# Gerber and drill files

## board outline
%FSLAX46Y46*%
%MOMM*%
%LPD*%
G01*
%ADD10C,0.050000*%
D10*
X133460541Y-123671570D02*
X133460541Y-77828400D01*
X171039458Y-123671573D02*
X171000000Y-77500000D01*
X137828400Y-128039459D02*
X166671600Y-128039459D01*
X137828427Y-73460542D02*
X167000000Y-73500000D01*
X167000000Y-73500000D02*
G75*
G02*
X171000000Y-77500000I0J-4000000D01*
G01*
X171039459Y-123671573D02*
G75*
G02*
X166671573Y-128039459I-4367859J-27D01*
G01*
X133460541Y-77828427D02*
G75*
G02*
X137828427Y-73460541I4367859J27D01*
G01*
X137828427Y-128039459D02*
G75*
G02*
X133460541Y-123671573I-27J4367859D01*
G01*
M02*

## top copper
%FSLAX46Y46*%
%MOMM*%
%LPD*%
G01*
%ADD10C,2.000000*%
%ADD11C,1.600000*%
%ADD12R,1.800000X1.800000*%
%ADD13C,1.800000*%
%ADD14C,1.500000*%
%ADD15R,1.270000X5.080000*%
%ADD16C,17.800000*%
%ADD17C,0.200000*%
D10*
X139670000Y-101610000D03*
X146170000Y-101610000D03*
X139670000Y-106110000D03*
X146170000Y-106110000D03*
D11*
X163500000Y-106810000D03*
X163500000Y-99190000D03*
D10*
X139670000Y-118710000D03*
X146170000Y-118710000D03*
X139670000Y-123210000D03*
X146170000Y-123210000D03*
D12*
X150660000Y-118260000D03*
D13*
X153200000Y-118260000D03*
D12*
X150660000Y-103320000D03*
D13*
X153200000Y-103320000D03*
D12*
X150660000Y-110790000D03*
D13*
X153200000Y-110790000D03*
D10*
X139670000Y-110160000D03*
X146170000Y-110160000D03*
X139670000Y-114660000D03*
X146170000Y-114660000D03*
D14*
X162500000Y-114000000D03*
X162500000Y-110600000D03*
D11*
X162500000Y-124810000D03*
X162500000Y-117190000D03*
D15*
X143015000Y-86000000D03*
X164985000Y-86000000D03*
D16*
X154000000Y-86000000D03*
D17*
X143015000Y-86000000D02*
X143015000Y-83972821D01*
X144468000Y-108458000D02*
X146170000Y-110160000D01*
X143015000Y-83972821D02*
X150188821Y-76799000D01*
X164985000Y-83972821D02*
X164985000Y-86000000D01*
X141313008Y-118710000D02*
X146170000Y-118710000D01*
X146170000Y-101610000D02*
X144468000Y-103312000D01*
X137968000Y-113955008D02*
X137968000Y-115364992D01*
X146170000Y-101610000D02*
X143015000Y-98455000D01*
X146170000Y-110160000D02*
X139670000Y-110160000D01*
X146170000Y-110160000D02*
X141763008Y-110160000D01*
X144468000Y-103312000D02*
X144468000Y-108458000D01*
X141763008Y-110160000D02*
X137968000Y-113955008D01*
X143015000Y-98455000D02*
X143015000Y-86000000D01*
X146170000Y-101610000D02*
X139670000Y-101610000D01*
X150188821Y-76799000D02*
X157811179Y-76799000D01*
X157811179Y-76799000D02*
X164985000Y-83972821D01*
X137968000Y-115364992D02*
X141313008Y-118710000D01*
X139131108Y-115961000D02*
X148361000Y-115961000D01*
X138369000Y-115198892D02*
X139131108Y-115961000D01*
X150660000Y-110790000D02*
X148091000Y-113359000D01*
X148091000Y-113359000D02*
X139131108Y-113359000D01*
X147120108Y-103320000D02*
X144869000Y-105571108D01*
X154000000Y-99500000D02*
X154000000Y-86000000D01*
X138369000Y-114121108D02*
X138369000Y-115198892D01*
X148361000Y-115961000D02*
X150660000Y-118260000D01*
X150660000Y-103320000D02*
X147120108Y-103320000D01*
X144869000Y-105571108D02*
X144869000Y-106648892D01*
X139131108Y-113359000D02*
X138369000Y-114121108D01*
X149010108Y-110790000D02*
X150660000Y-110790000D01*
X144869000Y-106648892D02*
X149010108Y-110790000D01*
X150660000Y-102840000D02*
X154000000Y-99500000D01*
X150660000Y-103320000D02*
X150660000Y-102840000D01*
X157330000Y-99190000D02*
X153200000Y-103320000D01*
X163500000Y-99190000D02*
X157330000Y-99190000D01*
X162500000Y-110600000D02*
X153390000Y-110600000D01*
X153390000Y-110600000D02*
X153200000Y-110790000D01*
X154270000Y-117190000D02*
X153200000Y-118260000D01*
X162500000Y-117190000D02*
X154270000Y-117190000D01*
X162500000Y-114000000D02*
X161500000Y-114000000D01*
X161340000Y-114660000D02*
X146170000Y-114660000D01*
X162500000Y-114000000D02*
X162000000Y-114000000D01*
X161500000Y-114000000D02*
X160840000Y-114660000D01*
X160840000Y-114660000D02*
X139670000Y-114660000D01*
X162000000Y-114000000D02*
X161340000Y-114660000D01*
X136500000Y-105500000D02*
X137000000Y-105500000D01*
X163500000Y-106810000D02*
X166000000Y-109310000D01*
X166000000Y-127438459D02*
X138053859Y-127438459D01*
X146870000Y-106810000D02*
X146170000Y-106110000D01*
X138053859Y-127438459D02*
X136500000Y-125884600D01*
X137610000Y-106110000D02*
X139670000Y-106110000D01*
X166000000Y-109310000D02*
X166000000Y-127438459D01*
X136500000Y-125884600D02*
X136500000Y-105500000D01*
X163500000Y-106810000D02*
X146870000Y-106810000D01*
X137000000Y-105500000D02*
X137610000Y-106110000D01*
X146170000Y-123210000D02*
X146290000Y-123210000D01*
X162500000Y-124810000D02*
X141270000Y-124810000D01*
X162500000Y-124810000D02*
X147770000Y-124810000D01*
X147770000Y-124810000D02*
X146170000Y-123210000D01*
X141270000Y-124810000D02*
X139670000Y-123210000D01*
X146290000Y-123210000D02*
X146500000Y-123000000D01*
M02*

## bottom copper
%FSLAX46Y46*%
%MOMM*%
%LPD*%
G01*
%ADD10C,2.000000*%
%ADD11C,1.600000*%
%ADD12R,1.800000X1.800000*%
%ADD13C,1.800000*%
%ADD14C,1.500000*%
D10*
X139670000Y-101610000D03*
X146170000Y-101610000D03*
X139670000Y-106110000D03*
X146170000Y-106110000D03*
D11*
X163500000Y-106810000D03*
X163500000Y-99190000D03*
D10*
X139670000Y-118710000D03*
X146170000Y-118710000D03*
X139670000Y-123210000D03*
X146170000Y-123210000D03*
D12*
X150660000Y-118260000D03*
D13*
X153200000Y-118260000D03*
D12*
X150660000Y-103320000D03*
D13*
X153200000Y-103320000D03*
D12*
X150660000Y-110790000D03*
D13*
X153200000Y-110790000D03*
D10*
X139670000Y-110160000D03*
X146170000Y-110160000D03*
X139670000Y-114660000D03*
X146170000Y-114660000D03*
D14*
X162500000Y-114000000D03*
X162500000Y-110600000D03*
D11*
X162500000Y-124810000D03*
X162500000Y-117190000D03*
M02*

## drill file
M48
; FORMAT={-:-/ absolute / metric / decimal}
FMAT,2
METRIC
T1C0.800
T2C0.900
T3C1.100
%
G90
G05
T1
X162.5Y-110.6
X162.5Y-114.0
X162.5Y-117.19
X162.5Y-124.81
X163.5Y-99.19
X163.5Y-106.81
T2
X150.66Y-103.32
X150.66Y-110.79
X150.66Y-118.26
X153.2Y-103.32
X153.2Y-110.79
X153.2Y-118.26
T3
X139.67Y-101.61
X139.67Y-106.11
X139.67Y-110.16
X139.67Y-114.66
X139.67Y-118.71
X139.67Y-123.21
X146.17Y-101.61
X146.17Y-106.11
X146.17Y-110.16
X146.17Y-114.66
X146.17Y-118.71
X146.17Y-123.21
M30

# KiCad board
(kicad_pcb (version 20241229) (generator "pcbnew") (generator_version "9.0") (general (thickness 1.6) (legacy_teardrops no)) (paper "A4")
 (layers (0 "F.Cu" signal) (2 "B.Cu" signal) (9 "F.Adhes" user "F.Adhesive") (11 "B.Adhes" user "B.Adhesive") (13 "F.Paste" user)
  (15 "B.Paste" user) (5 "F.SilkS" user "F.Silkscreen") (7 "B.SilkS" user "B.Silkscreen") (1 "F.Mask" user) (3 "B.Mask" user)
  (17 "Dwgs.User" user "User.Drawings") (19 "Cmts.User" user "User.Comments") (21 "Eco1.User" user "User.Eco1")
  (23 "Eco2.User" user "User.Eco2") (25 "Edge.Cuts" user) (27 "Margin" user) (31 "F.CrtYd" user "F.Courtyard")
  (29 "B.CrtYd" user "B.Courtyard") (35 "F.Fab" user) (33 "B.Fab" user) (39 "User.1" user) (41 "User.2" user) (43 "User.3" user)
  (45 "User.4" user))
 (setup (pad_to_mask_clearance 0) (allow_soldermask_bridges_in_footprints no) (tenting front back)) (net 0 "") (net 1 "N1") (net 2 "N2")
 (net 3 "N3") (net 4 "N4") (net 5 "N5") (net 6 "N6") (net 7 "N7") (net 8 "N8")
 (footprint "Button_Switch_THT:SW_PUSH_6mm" (layer "F.Cu") (at 139.67 101.61)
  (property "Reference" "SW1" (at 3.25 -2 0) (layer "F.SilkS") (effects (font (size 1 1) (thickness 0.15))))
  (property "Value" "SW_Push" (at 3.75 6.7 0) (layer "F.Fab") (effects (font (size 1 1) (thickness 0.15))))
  (pad "1" thru_hole circle (at 0 0 90) (size 2 2) (drill 1.1) (layers "*.Cu" "*.Mask") (remove_unused_layers no) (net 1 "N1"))
  (pad "1" thru_hole circle (at 6.5 0 90) (size 2 2) (drill 1.1) (layers "*.Cu" "*.Mask") (remove_unused_layers no) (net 1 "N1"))
  (pad "2" thru_hole circle (at 0 4.5 90) (size 2 2) (drill 1.1) (layers "*.Cu" "*.Mask") (remove_unused_layers no) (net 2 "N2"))
  (pad "2" thru_hole circle (at 6.5 4.5 90) (size 2 2) (drill 1.1) (layers "*.Cu" "*.Mask") (remove_unused_layers no) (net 2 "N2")))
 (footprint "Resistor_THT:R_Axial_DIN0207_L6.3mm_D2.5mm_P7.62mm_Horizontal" (layer "F.Cu") (at 163.5 106.81 90)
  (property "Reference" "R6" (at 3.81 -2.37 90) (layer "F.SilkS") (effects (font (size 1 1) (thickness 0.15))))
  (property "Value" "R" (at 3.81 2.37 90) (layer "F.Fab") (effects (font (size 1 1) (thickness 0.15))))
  (pad "1" thru_hole circle (at 0 0 90) (size 1.6 1.6) (drill 0.8) (layers "*.Cu" "*.Mask") (remove_unused_layers no) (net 2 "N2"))
  (pad "2" thru_hole circle (at 7.62 0 90) (size 1.6 1.6) (drill 0.8) (layers "*.Cu" "*.Mask") (remove_unused_layers no) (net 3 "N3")))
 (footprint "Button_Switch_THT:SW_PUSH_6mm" (layer "F.Cu") (at 139.67 118.71)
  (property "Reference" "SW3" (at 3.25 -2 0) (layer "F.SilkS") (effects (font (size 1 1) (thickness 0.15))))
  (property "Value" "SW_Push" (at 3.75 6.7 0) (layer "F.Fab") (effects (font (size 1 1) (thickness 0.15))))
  (pad "1" thru_hole circle (at 0 0 90) (size 2 2) (drill 1.1) (layers "*.Cu" "*.Mask") (remove_unused_layers no) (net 1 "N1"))
  (pad "1" thru_hole circle (at 6.5 0 90) (size 2 2) (drill 1.1) (layers "*.Cu" "*.Mask") (remove_unused_layers no) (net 1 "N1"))
  (pad "2" thru_hole circle (at 0 4.5 90) (size 2 2) (drill 1.1) (layers "*.Cu" "*.Mask") (remove_unused_layers no) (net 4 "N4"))
  (pad "2" thru_hole circle (at 6.5 4.5 90) (size 2 2) (drill 1.1) (layers "*.Cu" "*.Mask") (remove_unused_layers no) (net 4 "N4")))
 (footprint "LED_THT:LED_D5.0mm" (layer "F.Cu") (at 150.66 118.26)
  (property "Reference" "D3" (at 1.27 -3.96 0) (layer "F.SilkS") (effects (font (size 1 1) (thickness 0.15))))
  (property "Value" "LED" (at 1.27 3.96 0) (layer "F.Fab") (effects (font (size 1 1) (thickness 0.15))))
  (pad "1" thru_hole rect (at 0 0) (size 1.8 1.8) (drill 0.9) (layers "*.Cu" "*.Mask") (remove_unused_layers no) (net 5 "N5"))
  (pad "2" thru_hole circle (at 2.54 0) (size 1.8 1.8) (drill 0.9) (layers "*.Cu" "*.Mask") (remove_unused_layers no) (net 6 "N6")))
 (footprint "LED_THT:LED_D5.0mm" (layer "F.Cu") (at 150.66 103.32)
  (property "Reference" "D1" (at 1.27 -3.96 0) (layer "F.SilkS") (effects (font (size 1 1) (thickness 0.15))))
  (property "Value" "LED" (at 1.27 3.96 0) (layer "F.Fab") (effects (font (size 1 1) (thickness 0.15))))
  (pad "1" thru_hole rect (at 0 0) (size 1.8 1.8) (drill 0.9) (layers "*.Cu" "*.Mask") (remove_unused_layers no) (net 5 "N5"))
  (pad "2" thru_hole circle (at 2.54 0) (size 1.8 1.8) (drill 0.9) (layers "*.Cu" "*.Mask") (remove_unused_layers no) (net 3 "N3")))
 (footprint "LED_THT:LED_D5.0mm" (layer "F.Cu") (at 150.66 110.79)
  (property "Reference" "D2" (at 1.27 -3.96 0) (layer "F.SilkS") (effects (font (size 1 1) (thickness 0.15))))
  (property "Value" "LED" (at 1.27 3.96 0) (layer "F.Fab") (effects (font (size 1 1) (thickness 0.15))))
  (pad "1" thru_hole rect (at 0 0) (size 1.8 1.8) (drill 0.9) (layers "*.Cu" "*.Mask") (remove_unused_layers no) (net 5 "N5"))
  (pad "2" thru_hole circle (at 2.54 0) (size 1.8 1.8) (drill 0.9) (layers "*.Cu" "*.Mask") (remove_unused_layers no) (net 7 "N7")))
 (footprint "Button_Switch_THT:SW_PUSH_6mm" (layer "F.Cu") (at 139.67 110.16)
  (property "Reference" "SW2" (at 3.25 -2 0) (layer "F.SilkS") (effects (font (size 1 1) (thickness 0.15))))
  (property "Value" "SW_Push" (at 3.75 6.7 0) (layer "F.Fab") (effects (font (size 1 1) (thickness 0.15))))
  (pad "1" thru_hole circle (at 0 0 90) (size 2 2) (drill 1.1) (layers "*.Cu" "*.Mask") (remove_unused_layers no) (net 1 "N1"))
  (pad "1" thru_hole circle (at 6.5 0 90) (size 2 2) (drill 1.1) (layers "*.Cu" "*.Mask") (remove_unused_layers no) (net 1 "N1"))
  (pad "2" thru_hole circle (at 0 4.5 90) (size 2 2) (drill 1.1) (layers "*.Cu" "*.Mask") (remove_unused_layers no) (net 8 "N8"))
  (pad "2" thru_hole circle (at 6.5 4.5 90) (size 2 2) (drill 1.1) (layers "*.Cu" "*.Mask") (remove_unused_layers no) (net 8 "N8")))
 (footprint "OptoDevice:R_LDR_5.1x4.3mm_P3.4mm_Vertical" (layer "F.Cu") (at 162.5 114 90)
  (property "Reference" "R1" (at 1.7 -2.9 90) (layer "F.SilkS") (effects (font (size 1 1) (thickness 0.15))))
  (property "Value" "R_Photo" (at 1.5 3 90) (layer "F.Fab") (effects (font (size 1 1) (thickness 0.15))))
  (pad "1" thru_hole circle (at 0 0 90) (size 1.5 1.5) (drill 0.8) (layers "*.Cu" "*.Mask") (remove_unused_layers no) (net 8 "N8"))
  (pad "2" thru_hole circle (at 3.4 0 90) (size 1.5 1.5) (drill 0.8) (layers "*.Cu" "*.Mask") (remove_unused_layers no) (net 7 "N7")))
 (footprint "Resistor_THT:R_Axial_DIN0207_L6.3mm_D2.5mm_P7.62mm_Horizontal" (layer "F.Cu") (at 162.5 124.81 90)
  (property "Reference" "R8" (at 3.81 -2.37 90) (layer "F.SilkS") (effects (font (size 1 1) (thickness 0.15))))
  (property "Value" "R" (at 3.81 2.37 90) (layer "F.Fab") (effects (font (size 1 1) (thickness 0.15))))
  (pad "1" thru_hole circle (at 0 0 90) (size 1.6 1.6) (drill 0.8) (layers "*.Cu" "*.Mask") (remove_unused_layers no) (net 4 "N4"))
  (pad "2" thru_hole circle (at 7.62 0 90) (size 1.6 1.6) (drill 0.8) (layers "*.Cu" "*.Mask") (remove_unused_layers no) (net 6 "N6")))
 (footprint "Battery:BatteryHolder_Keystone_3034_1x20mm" (layer "F.Cu") (at 154 86)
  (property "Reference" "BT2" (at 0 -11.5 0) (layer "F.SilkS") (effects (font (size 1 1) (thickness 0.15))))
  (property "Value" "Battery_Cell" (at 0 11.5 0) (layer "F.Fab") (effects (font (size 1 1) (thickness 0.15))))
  (pad "1" smd rect (at -10.985 0) (size 1.27 5.08) (layers "F.Cu" "F.Mask" "F.Paste") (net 1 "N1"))
  (pad "1" smd rect (at 10.985 0) (size 1.27 5.08) (layers "F.Cu" "F.Mask" "F.Paste") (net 1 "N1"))
  (pad "2" smd circle (at 0 0) (size 17.8 17.8) (layers "F.Cu" "F.Mask") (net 5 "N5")))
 (gr_line (start 133.460541 123.67157) (end 133.460541 77.8284) (stroke (width 0.05) (type default)) (layer "Edge.Cuts"))
 (gr_line (start 171.039458 123.671573) (end 171 77.5) (stroke (width 0.05) (type default)) (layer "Edge.Cuts"))
 (gr_line (start 137.8284 128.039459) (end 166.6716 128.039459) (stroke (width 0.05) (type default)) (layer "Edge.Cuts"))
 (gr_line (start 137.828427 73.460542) (end 167 73.5) (stroke (width 0.05) (type default)) (layer "Edge.Cuts"))
 (gr_arc (start 167 73.5) (mid 169.828427 74.671573) (end 171 77.5) (stroke (width 0.05) (type default)) (layer "Edge.Cuts"))
 (gr_arc (start 171.039459 123.671573) (mid 169.760135 126.760135) (end 166.671573 128.039459) (stroke (width 0.05) (type default))
  (layer "Edge.Cuts"))
 (gr_arc (start 133.460541 77.828427) (mid 134.739865 74.739865) (end 137.828427 73.460541) (stroke (width 0.05) (type default))
  (layer "Edge.Cuts"))
 (gr_arc (start 137.828427 128.039459) (mid 134.739865 126.760135) (end 133.460541 123.671573) (stroke (width 0.05) (type default))
  (layer "Edge.Cuts"))
 (segment (start 143.015 86) (end 143.015 83.972821) (width 0.2) (layer "F.Cu") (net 1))
 (segment (start 144.468 108.458) (end 146.17 110.16) (width 0.2) (layer "F.Cu") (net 1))
 (segment (start 143.015 83.972821) (end 150.188821 76.799) (width 0.2) (layer "F.Cu") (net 1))
 (segment (start 164.985 83.972821) (end 164.985 86) (width 0.2) (layer "F.Cu") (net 1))
 (segment (start 141.313008 118.71) (end 146.17 118.71) (width 0.2) (layer "F.Cu") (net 1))
 (segment (start 146.17 101.61) (end 144.468 103.312) (width 0.2) (layer "F.Cu") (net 1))
 (segment (start 137.968 113.955008) (end 137.968 115.364992) (width 0.2) (layer "F.Cu") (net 1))
 (segment (start 146.17 101.61) (end 143.015 98.455) (width 0.2) (layer "F.Cu") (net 1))
 (segment (start 146.17 110.16) (end 139.67 110.16) (width 0.2) (layer "F.Cu") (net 1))
 (segment (start 146.17 110.16) (end 141.763008 110.16) (width 0.2) (layer "F.Cu") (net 1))
 (segment (start 144.468 103.312) (end 144.468 108.458) (width 0.2) (layer "F.Cu") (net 1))
 (segment (start 141.763008 110.16) (end 137.968 113.955008) (width 0.2) (layer "F.Cu") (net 1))
 (segment (start 143.015 98.455) (end 143.015 86) (width 0.2) (layer "F.Cu") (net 1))
 (segment (start 146.17 101.61) (end 139.67 101.61) (width 0.2) (layer "F.Cu") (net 1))
 (segment (start 150.188821 76.799) (end 157.811179 76.799) (width 0.2) (layer "F.Cu") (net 1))
 (segment (start 157.811179 76.799) (end 164.985 83.972821) (width 0.2) (layer "F.Cu") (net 1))
 (segment (start 137.968 115.364992) (end 141.313008 118.71) (width 0.2) (layer "F.Cu") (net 1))
 (segment (start 139.131108 115.961) (end 148.361 115.961) (width 0.2) (layer "F.Cu") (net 5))
 (segment (start 138.369 115.198892) (end 139.131108 115.961) (width 0.2) (layer "F.Cu") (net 5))
 (segment (start 150.66 110.79) (end 148.091 113.359) (width 0.2) (layer "F.Cu") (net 5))
 (segment (start 148.091 113.359) (end 139.131108 113.359) (width 0.2) (layer "F.Cu") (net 5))
 (segment (start 147.120108 103.32) (end 144.869 105.571108) (width 0.2) (layer "F.Cu") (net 5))
 (segment (start 154 99.5) (end 154 86) (width 0.2) (layer "F.Cu") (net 5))
 (segment (start 138.369 114.121108) (end 138.369 115.198892) (width 0.2) (layer "F.Cu") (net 5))
 (segment (start 148.361 115.961) (end 150.66 118.26) (width 0.2) (layer "F.Cu") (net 5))
 (segment (start 150.66 103.32) (end 147.120108 103.32) (width 0.2) (layer "F.Cu") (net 5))
 (segment (start 144.869 105.571108) (end 144.869 106.648892) (width 0.2) (layer "F.Cu") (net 5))
 (segment (start 139.131108 113.359) (end 138.369 114.121108) (width 0.2) (layer "F.Cu") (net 5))
 (segment (start 149.010108 110.79) (end 150.66 110.79) (width 0.2) (layer "F.Cu") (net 5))
 (segment (start 144.869 106.648892) (end 149.010108 110.79) (width 0.2) (layer "F.Cu") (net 5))
 (segment (start 150.66 102.84) (end 154 99.5) (width 0.2) (layer "F.Cu") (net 5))
 (segment (start 150.66 103.32) (end 150.66 102.84) (width 0.2) (layer "F.Cu") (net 5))
 (segment (start 157.33 99.19) (end 153.2 103.32) (width 0.2) (layer "F.Cu") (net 3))
 (segment (start 163.5 99.19) (end 157.33 99.19) (width 0.2) (layer "F.Cu") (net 3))
 (segment (start 162.5 110.6) (end 153.39 110.6) (width 0.2) (layer "F.Cu") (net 7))
 (segment (start 153.39 110.6) (end 153.2 110.79) (width 0.2) (layer "F.Cu") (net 7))
 (segment (start 154.27 117.19) (end 153.2 118.26) (width 0.2) (layer "F.Cu") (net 6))
 (segment (start 162.5 117.19) (end 154.27 117.19) (width 0.2) (layer "F.Cu") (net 6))
 (segment (start 162.5 114) (end 161.5 114) (width 0.2) (layer "F.Cu") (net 8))
 (segment (start 161.34 114.66) (end 146.17 114.66) (width 0.2) (layer "F.Cu") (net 8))
 (segment (start 162.5 114) (end 162 114) (width 0.2) (layer "F.Cu") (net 8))
 (segment (start 161.5 114) (end 160.84 114.66) (width 0.2) (layer "F.Cu") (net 8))
 (segment (start 160.84 114.66) (end 139.67 114.66) (width 0.2) (layer "F.Cu") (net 8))
 (segment (start 162 114) (end 161.34 114.66) (width 0.2) (layer "F.Cu") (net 8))
 (segment (start 136.5 105.5) (end 137 105.5) (width 0.2) (layer "F.Cu") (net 2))
 (segment (start 163.5 106.81) (end 166 109.31) (width 0.2) (layer "F.Cu") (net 2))
 (segment (start 166 127.438459) (end 138.053859 127.438459) (width 0.2) (layer "F.Cu") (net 2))
 (segment (start 146.87 106.81) (end 146.17 106.11) (width 0.2) (layer "F.Cu") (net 2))
 (segment (start 138.053859 127.438459) (end 136.5 125.8846) (width 0.2) (layer "F.Cu") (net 2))
 (segment (start 137.61 106.11) (end 139.67 106.11) (width 0.2) (layer "F.Cu") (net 2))
 (segment (start 166 109.31) (end 166 127.438459) (width 0.2) (layer "F.Cu") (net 2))
 (segment (start 136.5 125.8846) (end 136.5 105.5) (width 0.2) (layer "F.Cu") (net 2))
 (segment (start 163.5 106.81) (end 146.87 106.81) (width 0.2) (layer "F.Cu") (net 2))
 (segment (start 137 105.5) (end 137.61 106.11) (width 0.2) (layer "F.Cu") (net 2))
 (segment (start 146.17 123.21) (end 146.29 123.21) (width 0.2) (layer "F.Cu") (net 4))
 (segment (start 162.5 124.81) (end 141.27 124.81) (width 0.2) (layer "F.Cu") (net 4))
 (segment (start 162.5 124.81) (end 147.77 124.81) (width 0.2) (layer "F.Cu") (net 4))
 (segment (start 147.77 124.81) (end 146.17 123.21) (width 0.2) (layer "F.Cu") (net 4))
 (segment (start 141.27 124.81) (end 139.67 123.21) (width 0.2) (layer "F.Cu") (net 4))
 (segment (start 146.29 123.21) (end 146.5 123) (width 0.2) (layer "F.Cu") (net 4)))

